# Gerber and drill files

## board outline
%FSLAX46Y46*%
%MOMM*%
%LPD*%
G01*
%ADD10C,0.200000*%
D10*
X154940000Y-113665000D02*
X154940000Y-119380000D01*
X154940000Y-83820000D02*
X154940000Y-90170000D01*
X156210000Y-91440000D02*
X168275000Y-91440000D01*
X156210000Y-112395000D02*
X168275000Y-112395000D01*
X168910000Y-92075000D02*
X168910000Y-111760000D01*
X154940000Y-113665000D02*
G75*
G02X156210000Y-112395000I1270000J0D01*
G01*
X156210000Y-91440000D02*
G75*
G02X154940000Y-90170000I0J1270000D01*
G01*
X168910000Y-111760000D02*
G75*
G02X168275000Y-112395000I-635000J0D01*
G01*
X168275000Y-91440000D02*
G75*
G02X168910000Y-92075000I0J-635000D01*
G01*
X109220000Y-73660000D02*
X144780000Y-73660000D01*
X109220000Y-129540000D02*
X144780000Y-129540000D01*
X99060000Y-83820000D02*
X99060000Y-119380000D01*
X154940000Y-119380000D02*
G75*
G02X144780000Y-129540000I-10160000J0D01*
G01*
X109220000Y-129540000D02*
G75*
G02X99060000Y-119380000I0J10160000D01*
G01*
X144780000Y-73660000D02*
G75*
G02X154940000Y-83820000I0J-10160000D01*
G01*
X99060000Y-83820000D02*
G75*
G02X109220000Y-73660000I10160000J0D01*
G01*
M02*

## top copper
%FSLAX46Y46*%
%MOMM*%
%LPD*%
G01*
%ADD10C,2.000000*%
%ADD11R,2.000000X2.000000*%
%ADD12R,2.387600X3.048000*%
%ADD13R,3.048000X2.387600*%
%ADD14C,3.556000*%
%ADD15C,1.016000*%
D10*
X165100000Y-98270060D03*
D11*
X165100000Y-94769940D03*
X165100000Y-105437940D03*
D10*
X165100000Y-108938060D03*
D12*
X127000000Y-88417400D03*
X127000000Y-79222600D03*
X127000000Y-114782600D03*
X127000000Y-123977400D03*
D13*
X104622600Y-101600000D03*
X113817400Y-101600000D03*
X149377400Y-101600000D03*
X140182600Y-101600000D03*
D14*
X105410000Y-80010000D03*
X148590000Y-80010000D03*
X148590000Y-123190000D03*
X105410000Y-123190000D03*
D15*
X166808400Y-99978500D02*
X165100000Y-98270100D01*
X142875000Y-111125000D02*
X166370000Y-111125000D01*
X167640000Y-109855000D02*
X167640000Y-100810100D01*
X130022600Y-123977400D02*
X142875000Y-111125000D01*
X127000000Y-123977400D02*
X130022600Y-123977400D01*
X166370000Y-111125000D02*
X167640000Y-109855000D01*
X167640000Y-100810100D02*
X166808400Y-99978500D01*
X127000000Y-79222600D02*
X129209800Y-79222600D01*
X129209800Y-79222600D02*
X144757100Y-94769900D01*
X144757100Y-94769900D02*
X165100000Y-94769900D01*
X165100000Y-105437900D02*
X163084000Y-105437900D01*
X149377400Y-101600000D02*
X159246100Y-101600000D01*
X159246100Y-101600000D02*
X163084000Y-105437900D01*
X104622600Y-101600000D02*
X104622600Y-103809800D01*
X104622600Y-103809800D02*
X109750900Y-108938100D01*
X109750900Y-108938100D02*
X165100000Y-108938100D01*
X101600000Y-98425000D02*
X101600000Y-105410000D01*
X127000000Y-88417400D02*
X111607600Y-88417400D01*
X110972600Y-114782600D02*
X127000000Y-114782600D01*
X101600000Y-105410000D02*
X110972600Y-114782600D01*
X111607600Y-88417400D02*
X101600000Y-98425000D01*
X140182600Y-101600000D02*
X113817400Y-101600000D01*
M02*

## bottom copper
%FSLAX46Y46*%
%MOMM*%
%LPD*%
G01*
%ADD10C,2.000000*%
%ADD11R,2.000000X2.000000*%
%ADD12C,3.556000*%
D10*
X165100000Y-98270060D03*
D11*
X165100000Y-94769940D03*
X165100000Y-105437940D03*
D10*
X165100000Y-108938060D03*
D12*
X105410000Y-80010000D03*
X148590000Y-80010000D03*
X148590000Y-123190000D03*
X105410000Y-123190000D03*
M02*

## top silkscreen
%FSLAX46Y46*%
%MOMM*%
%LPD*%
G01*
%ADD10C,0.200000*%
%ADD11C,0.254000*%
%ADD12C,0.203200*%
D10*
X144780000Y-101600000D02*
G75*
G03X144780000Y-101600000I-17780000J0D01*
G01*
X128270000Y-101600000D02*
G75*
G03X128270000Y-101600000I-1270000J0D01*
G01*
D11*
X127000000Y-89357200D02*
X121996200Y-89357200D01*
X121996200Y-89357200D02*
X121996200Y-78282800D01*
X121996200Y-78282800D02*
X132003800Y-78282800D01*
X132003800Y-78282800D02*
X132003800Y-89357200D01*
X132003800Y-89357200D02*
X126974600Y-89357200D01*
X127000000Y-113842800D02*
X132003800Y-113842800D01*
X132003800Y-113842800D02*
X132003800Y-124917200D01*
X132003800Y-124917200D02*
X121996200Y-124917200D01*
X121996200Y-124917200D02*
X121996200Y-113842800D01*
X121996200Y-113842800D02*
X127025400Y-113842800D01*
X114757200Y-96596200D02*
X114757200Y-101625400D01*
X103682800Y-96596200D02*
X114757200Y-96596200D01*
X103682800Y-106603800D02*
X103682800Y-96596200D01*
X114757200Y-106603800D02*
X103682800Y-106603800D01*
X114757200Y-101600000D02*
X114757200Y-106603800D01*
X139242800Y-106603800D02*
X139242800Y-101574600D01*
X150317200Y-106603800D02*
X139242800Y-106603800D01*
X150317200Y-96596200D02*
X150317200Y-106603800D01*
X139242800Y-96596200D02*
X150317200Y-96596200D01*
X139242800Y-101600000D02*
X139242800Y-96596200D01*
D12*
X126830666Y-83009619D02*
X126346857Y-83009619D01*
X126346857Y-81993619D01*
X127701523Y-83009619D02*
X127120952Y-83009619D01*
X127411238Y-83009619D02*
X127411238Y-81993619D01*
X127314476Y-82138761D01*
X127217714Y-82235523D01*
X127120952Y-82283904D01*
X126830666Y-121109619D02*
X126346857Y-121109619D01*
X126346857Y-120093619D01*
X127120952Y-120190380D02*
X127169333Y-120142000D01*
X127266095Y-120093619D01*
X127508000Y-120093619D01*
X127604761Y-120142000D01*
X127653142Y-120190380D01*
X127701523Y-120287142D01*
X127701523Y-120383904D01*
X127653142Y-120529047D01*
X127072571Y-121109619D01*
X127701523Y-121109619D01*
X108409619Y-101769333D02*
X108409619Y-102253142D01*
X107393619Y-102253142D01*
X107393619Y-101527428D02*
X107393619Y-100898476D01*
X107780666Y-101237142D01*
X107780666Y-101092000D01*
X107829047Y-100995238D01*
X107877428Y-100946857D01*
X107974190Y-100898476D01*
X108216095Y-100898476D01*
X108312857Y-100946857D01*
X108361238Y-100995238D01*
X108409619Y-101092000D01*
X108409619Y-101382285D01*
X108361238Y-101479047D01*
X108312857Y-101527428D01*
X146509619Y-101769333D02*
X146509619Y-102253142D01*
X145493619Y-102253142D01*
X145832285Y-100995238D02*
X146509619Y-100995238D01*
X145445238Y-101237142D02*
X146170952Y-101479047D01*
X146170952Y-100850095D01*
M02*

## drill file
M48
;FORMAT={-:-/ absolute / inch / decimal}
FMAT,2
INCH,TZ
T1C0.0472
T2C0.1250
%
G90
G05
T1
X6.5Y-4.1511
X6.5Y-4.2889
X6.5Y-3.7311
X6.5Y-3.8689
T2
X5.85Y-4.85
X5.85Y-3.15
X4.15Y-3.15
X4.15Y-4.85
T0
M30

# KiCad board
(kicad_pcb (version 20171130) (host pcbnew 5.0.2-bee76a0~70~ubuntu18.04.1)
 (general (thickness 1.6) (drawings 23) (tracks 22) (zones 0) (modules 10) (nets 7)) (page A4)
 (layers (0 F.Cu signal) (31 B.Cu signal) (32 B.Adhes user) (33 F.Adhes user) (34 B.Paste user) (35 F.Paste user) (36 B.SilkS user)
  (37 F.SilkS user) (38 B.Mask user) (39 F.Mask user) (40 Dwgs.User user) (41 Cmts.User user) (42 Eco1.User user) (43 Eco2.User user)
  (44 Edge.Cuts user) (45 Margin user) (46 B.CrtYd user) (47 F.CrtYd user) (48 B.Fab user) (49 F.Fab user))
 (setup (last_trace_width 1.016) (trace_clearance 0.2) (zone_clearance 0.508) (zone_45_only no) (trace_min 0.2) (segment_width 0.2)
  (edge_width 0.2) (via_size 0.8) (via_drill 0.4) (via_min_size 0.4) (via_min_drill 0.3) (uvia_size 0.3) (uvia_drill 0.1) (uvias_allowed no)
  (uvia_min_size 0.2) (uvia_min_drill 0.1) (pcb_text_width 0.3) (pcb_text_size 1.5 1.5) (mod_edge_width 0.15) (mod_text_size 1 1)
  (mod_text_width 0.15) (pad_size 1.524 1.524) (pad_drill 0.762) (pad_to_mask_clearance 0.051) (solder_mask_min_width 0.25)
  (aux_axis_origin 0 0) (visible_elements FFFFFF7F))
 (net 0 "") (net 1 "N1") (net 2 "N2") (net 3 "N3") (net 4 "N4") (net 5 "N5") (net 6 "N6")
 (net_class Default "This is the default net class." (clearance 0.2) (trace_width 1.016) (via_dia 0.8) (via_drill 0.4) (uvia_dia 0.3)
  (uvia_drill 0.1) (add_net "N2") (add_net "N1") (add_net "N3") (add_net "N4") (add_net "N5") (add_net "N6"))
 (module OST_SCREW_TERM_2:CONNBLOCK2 (layer B.Cu) (at 165.1 96.52 270)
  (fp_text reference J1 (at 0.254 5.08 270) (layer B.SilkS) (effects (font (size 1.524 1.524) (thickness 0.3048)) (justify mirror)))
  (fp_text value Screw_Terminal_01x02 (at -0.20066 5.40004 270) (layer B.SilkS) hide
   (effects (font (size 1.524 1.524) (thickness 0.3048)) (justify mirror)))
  (pad 2 thru_hole circle (at 1.75006 0 270) (size 2 2) (drill 1.2) (layers *.Cu *.Mask) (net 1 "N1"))
  (pad 1 thru_hole rect (at -1.75006 0 270) (size 2 2) (drill 1.2) (layers *.Cu *.Mask) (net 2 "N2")))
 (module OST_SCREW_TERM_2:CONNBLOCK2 (layer B.Cu) (at 165.1 107.188 270)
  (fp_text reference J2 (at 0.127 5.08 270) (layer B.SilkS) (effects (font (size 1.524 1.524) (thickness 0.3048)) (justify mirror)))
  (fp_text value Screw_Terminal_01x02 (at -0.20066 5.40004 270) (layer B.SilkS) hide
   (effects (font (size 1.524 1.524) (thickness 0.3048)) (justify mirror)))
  (pad 1 thru_hole rect (at -1.75006 0 270) (size 2 2) (drill 1.2) (layers *.Cu *.Mask) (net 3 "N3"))
  (pad 2 thru_hole circle (at 1.75006 0 270) (size 2 2) (drill 1.2) (layers *.Cu *.Mask) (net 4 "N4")))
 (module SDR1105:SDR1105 (layer F.Cu) (at 127 83.82 180)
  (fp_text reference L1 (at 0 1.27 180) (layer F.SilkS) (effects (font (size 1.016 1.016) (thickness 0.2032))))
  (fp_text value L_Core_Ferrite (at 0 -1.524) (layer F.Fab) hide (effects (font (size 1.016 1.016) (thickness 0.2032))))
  (fp_line (start 0 -5.5372) (end 5.0038 -5.5372) (layer F.SilkS) (width 0.254))
  (fp_line (start 5.0038 -5.5372) (end 5.0038 5.5372) (layer F.SilkS) (width 0.254))
  (fp_line (start 5.0038 5.5372) (end -5.0038 5.5372) (layer F.SilkS) (width 0.254))
  (fp_line (start -5.0038 5.5372) (end -5.0038 -5.5372) (layer F.SilkS) (width 0.254))
  (fp_line (start -5.0038 -5.5372) (end 0.0254 -5.5372) (layer F.SilkS) (width 0.254))
  (pad 1 smd rect (at 0 -4.5974 180) (size 2.3876 3.048) (layers F.Cu F.Paste F.Mask) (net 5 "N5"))
  (pad 2 smd rect (at 0 4.5974 180) (size 2.3876 3.048) (layers F.Cu F.Paste F.Mask) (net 2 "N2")))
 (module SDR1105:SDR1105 (layer F.Cu) (at 127 119.38)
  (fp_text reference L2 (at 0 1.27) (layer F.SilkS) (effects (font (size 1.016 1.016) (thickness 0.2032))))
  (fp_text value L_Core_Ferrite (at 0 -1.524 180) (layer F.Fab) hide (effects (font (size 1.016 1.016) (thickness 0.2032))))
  (fp_line (start 0 -5.5372) (end 5.0038 -5.5372) (layer F.SilkS) (width 0.254))
  (fp_line (start 5.0038 -5.5372) (end 5.0038 5.5372) (layer F.SilkS) (width 0.254))
  (fp_line (start 5.0038 5.5372) (end -5.0038 5.5372) (layer F.SilkS) (width 0.254))
  (fp_line (start -5.0038 5.5372) (end -5.0038 -5.5372) (layer F.SilkS) (width 0.254))
  (fp_line (start -5.0038 -5.5372) (end 0.0254 -5.5372) (layer F.SilkS) (width 0.254))
  (pad 1 smd rect (at 0 -4.5974) (size 2.3876 3.048) (layers F.Cu F.Paste F.Mask) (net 5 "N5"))
  (pad 2 smd rect (at 0 4.5974) (size 2.3876 3.048) (layers F.Cu F.Paste F.Mask) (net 1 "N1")))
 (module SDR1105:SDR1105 (layer F.Cu) (at 109.22 101.6 270)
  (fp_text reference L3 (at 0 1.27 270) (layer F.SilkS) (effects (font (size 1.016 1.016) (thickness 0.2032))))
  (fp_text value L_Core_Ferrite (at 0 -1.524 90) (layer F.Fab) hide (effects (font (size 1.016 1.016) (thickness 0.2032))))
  (fp_line (start -5.0038 -5.5372) (end 0.0254 -5.5372) (layer F.SilkS) (width 0.254))
  (fp_line (start -5.0038 5.5372) (end -5.0038 -5.5372) (layer F.SilkS) (width 0.254))
  (fp_line (start 5.0038 5.5372) (end -5.0038 5.5372) (layer F.SilkS) (width 0.254))
  (fp_line (start 5.0038 -5.5372) (end 5.0038 5.5372) (layer F.SilkS) (width 0.254))
  (fp_line (start 0 -5.5372) (end 5.0038 -5.5372) (layer F.SilkS) (width 0.254))
  (pad 2 smd rect (at 0 4.5974 270) (size 2.3876 3.048) (layers F.Cu F.Paste F.Mask) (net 4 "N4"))
  (pad 1 smd rect (at 0 -4.5974 270) (size 2.3876 3.048) (layers F.Cu F.Paste F.Mask) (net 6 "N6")))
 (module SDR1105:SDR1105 (layer F.Cu) (at 144.78 101.6 90)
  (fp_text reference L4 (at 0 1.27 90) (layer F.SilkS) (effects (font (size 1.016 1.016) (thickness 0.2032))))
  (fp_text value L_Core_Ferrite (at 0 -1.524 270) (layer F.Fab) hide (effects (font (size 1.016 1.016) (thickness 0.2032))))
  (fp_line (start -5.0038 -5.5372) (end 0.0254 -5.5372) (layer F.SilkS) (width 0.254))
  (fp_line (start -5.0038 5.5372) (end -5.0038 -5.5372) (layer F.SilkS) (width 0.254))
  (fp_line (start 5.0038 5.5372) (end -5.0038 5.5372) (layer F.SilkS) (width 0.254))
  (fp_line (start 5.0038 -5.5372) (end 5.0038 5.5372) (layer F.SilkS) (width 0.254))
  (fp_line (start 0 -5.5372) (end 5.0038 -5.5372) (layer F.SilkS) (width 0.254))
  (pad 2 smd rect (at 0 4.5974 90) (size 2.3876 3.048) (layers F.Cu F.Paste F.Mask) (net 3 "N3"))
  (pad 1 smd rect (at 0 -4.5974 90) (size 2.3876 3.048) (layers F.Cu F.Paste F.Mask) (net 6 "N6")))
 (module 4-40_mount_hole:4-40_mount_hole (layer F.Cu) (at 105.41 80.01)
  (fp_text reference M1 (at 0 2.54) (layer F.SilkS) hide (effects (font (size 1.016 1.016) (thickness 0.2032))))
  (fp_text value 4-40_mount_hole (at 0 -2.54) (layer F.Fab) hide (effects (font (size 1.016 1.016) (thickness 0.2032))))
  (pad "" thru_hole circle (at 0 0) (size 3.556 3.556) (drill 3.175) (layers *.Cu *.Mask)))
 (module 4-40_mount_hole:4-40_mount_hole (layer F.Cu) (at 148.59 80.01)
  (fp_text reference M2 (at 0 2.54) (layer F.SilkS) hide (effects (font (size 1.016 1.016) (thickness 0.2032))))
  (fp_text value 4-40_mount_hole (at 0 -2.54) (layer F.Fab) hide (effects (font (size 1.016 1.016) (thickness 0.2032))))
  (pad "" thru_hole circle (at 0 0) (size 3.556 3.556) (drill 3.175) (layers *.Cu *.Mask)))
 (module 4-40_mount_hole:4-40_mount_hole (layer F.Cu) (at 148.59 123.19)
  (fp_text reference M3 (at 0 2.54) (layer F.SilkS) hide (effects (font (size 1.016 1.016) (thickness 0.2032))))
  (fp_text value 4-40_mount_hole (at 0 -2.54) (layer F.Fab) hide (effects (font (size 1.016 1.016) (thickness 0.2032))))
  (pad "" thru_hole circle (at 0 0) (size 3.556 3.556) (drill 3.175) (layers *.Cu *.Mask)))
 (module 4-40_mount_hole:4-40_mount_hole (layer F.Cu) (at 105.41 123.19)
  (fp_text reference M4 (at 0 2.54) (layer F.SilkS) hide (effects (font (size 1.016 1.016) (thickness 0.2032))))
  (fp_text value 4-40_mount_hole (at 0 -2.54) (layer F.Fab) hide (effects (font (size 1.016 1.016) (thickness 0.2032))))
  (pad "" thru_hole circle (at 0 0) (size 3.556 3.556) (drill 3.175) (layers *.Cu *.Mask)))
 (gr_line (start 154.94 113.665) (end 154.94 119.38) (layer Edge.Cuts) (width 0.2))
 (gr_line (start 154.94 83.82) (end 154.94 90.17) (layer Edge.Cuts) (width 0.2))
 (gr_line (start 156.21 91.44) (end 168.275 91.44) (layer Edge.Cuts) (width 0.2))
 (gr_line (start 156.21 112.395) (end 168.275 112.395) (layer Edge.Cuts) (width 0.2))
 (gr_line (start 168.91 92.075) (end 168.91 111.76) (layer Edge.Cuts) (width 0.2))
 (gr_circle (center 127 101.6) (end 127 83.82) (layer F.SilkS) (width 0.2))
 (gr_circle (center 127 101.6) (end 128.27 101.6) (layer F.SilkS) (width 0.2))
 (gr_arc (start 156.21 113.665) (end 156.21 112.395) (angle -90) (layer Edge.Cuts) (width 0.2))
 (gr_arc (start 156.21 90.17) (end 154.94 90.17) (angle -90) (layer Edge.Cuts) (width 0.2))
 (gr_arc (start 168.275 111.76) (end 168.275 112.395) (angle -90) (layer Edge.Cuts) (width 0.2))
 (gr_arc (start 168.275 92.075) (end 168.91 92.075) (angle -90) (layer Edge.Cuts) (width 0.2))
 (gr_line (start 109.22 73.66) (end 144.78 73.66) (layer Edge.Cuts) (width 0.2))
 (gr_line (start 109.22 129.54) (end 144.78 129.54) (layer Edge.Cuts) (width 0.2))
 (gr_line (start 99.06 83.82) (end 99.06 119.38) (layer Edge.Cuts) (width 0.2))
 (gr_arc (start 144.78 119.38) (end 144.78 129.54) (angle -90) (layer Edge.Cuts) (width 0.2))
 (gr_arc (start 109.22 119.38) (end 99.06 119.38) (angle -90) (layer Edge.Cuts) (width 0.2))
 (gr_arc (start 144.78 83.82) (end 154.94 83.82) (angle -90) (layer Edge.Cuts) (width 0.2))
 (gr_arc (start 109.22 83.82) (end 109.22 73.66) (angle -90) (layer Edge.Cuts) (width 0.2))
 (segment (start 166.8084 99.9785) (end 165.1 98.2701) (width 1.016) (layer F.Cu) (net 1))
 (segment (start 142.875 111.125) (end 166.37 111.125) (width 1.016) (layer F.Cu) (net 1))
 (segment (start 167.64 109.855) (end 167.64 100.8101) (width 1.016) (layer F.Cu) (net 1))
 (segment (start 130.0226 123.9774) (end 142.875 111.125) (width 1.016) (layer F.Cu) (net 1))
 (segment (start 127 123.9774) (end 130.0226 123.9774) (width 1.016) (layer F.Cu) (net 1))
 (segment (start 166.37 111.125) (end 167.64 109.855) (width 1.016) (layer F.Cu) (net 1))
 (segment (start 167.64 100.8101) (end 166.8084 99.9785) (width 1.016) (layer F.Cu) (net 1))
 (segment (start 127 79.2226) (end 129.2098 79.2226) (width 1.016) (layer F.Cu) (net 2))
 (segment (start 129.2098 79.2226) (end 144.7571 94.7699) (width 1.016) (layer F.Cu) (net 2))
 (segment (start 144.7571 94.7699) (end 165.1 94.7699) (width 1.016) (layer F.Cu) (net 2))
 (segment (start 165.1 105.4379) (end 163.084 105.4379) (width 1.016) (layer F.Cu) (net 3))
 (segment (start 149.3774 101.6) (end 159.2461 101.6) (width 1.016) (layer F.Cu) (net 3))
 (segment (start 159.2461 101.6) (end 163.084 105.4379) (width 1.016) (layer F.Cu) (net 3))
 (segment (start 104.6226 101.6) (end 104.6226 103.8098) (width 1.016) (layer F.Cu) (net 4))
 (segment (start 104.6226 103.8098) (end 109.7509 108.9381) (width 1.016) (layer F.Cu) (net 4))
 (segment (start 109.7509 108.9381) (end 165.1 108.9381) (width 1.016) (layer F.Cu) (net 4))
 (segment (start 101.6 98.425) (end 101.6 105.41) (width 1.016) (layer F.Cu) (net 5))
 (segment (start 127 88.4174) (end 111.6076 88.4174) (width 1.016) (layer F.Cu) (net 5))
 (segment (start 110.9726 114.7826) (end 127 114.7826) (width 1.016) (layer F.Cu) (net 5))
 (segment (start 101.6 105.41) (end 110.9726 114.7826) (width 1.016) (layer F.Cu) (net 5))
 (segment (start 111.6076 88.4174) (end 101.6 98.425) (width 1.016) (layer F.Cu) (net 5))
 (segment (start 140.1826 101.6) (end 113.8174 101.6) (width 1.016) (layer F.Cu) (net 6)))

